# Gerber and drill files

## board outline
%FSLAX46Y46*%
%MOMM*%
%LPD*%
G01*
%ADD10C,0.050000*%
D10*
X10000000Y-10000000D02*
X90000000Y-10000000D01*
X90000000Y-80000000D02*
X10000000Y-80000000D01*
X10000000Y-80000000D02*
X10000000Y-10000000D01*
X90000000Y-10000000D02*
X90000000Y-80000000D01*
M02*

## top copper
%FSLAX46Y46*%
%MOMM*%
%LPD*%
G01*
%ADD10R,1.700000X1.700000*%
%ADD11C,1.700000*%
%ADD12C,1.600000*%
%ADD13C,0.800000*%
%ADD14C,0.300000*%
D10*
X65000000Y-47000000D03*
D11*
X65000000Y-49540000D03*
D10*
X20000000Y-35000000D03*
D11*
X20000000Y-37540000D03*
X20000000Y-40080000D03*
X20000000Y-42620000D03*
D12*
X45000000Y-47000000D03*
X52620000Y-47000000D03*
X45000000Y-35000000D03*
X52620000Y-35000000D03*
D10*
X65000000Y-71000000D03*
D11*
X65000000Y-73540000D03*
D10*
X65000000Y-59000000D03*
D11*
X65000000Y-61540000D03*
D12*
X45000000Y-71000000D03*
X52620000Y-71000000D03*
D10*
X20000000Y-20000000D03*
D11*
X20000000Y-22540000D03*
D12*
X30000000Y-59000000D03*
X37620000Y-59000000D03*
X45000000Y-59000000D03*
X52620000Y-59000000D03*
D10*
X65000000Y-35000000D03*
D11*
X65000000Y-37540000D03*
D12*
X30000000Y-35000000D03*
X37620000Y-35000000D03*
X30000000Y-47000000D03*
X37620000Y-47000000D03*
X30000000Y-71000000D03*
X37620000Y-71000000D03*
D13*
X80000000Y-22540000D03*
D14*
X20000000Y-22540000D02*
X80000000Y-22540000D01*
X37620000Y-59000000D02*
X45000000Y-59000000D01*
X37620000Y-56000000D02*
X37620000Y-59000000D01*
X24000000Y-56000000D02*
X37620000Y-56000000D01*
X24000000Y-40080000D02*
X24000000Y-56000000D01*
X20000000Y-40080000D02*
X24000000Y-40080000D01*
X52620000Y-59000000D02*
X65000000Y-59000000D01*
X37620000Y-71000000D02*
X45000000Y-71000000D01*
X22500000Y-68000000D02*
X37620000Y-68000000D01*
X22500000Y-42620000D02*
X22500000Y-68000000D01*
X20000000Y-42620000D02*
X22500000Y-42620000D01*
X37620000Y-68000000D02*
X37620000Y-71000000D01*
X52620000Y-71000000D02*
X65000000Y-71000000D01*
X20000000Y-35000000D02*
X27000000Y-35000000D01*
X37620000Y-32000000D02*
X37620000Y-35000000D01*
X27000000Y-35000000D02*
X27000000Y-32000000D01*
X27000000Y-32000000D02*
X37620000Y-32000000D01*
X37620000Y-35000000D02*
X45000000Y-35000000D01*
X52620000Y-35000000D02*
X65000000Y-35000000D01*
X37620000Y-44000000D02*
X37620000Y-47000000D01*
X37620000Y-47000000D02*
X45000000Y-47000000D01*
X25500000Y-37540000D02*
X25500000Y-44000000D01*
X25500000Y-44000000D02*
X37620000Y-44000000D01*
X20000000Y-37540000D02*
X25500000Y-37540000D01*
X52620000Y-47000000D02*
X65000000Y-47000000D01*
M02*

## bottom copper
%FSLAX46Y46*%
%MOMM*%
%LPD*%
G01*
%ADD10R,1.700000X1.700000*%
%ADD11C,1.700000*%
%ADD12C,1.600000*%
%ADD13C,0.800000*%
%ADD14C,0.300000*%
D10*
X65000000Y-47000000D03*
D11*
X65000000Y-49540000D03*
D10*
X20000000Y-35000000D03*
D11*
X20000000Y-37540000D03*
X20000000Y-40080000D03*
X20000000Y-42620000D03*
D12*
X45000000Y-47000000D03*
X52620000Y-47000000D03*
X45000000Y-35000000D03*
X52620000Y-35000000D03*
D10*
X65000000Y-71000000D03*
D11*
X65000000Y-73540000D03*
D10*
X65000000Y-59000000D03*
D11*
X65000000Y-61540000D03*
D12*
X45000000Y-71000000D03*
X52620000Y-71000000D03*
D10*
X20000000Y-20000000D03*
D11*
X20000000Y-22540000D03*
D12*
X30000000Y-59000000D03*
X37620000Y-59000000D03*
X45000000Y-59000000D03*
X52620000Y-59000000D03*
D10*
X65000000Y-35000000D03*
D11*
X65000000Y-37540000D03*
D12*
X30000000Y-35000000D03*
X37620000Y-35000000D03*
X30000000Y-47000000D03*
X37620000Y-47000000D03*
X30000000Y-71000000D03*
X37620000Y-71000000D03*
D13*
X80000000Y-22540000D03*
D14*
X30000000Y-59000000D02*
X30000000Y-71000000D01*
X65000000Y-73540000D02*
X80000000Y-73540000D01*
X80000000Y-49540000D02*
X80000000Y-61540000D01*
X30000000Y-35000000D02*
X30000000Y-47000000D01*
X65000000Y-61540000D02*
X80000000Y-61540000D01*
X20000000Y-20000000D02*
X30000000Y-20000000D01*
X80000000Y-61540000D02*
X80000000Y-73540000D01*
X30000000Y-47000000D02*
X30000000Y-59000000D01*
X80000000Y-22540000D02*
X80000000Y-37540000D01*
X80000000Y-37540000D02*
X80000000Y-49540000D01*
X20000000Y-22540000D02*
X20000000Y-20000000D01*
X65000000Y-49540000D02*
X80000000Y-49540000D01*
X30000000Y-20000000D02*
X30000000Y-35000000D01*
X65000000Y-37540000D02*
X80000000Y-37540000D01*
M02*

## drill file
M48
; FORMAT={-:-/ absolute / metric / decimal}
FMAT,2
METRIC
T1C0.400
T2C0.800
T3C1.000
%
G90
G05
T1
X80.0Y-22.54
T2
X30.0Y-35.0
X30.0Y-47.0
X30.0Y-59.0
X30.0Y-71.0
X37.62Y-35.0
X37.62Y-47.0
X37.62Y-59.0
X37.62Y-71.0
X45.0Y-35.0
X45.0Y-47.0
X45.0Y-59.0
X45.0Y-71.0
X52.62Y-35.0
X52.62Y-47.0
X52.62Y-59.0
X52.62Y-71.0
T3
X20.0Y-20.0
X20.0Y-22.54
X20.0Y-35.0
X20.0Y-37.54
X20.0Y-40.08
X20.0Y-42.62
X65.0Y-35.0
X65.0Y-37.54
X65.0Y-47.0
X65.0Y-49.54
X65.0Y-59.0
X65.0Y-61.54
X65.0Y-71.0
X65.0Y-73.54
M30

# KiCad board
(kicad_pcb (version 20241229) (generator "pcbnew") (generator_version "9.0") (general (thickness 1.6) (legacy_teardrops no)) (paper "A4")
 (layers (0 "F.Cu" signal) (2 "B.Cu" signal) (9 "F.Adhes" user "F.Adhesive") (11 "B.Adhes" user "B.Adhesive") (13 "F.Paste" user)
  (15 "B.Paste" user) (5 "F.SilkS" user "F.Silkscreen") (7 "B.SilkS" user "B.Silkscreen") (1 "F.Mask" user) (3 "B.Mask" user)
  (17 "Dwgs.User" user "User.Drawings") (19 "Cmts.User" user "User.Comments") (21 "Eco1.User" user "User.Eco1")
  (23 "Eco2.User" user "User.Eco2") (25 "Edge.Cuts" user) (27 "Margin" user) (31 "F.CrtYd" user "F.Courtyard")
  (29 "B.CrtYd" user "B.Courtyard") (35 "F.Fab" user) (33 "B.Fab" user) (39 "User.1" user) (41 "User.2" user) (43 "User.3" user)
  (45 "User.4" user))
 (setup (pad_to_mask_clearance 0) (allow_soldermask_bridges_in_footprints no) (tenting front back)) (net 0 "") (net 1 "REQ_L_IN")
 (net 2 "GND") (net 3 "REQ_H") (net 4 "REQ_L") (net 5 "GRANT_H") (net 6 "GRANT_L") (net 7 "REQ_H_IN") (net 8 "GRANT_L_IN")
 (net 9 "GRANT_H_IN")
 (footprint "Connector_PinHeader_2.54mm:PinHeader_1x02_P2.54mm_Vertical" (layer "F.Cu") (at 65 47)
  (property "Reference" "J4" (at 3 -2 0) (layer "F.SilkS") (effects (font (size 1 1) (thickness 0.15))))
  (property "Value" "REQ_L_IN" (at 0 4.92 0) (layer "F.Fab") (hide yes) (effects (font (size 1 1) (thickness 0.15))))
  (pad "1" thru_hole rect (at 0 0) (size 1.7 1.7) (drill 1) (layers "*.Cu" "*.Mask") (remove_unused_layers no) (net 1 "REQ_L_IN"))
  (pad "2" thru_hole circle (at 0 2.54) (size 1.7 1.7) (drill 1) (layers "*.Cu" "*.Mask") (remove_unused_layers no) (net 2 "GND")))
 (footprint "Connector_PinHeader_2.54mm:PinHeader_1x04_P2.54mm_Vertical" (layer "F.Cu") (at 20 35)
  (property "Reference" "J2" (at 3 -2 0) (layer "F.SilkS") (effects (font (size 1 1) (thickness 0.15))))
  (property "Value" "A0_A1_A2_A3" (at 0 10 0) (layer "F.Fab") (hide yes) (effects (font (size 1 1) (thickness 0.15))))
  (pad "1" thru_hole rect (at 0 0) (size 1.7 1.7) (drill 1) (layers "*.Cu" "*.Mask") (remove_unused_layers no) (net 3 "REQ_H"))
  (pad "2" thru_hole circle (at 0 2.54) (size 1.7 1.7) (drill 1) (layers "*.Cu" "*.Mask") (remove_unused_layers no) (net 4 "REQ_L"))
  (pad "3" thru_hole circle (at 0 5.08) (size 1.7 1.7) (drill 1) (layers "*.Cu" "*.Mask") (remove_unused_layers no) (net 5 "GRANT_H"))
  (pad "4" thru_hole circle (at 0 7.62) (size 1.7 1.7) (drill 1) (layers "*.Cu" "*.Mask") (remove_unused_layers no) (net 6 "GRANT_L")))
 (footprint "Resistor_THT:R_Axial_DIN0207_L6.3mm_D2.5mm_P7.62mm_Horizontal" (layer "F.Cu") (at 45 47)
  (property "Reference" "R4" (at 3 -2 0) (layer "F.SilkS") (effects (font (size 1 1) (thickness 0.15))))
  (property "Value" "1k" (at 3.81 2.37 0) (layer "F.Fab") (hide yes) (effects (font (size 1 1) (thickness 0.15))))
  (pad "1" thru_hole circle (at 0 0) (size 1.6 1.6) (drill 0.8) (layers "*.Cu" "*.Mask") (remove_unused_layers no) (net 4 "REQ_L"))
  (pad "2" thru_hole circle (at 7.62 0) (size 1.6 1.6) (drill 0.8) (layers "*.Cu" "*.Mask") (remove_unused_layers no) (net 1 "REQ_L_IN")))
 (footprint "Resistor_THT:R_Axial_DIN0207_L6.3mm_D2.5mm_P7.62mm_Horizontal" (layer "F.Cu") (at 45 35)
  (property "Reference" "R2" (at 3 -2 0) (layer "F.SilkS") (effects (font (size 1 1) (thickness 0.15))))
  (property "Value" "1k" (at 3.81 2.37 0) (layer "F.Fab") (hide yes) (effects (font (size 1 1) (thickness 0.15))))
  (pad "1" thru_hole circle (at 0 0) (size 1.6 1.6) (drill 0.8) (layers "*.Cu" "*.Mask") (remove_unused_layers no) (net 3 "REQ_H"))
  (pad "2" thru_hole circle (at 7.62 0) (size 1.6 1.6) (drill 0.8) (layers "*.Cu" "*.Mask") (remove_unused_layers no) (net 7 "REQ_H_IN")))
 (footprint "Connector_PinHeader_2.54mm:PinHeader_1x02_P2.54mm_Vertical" (layer "F.Cu") (at 65 71)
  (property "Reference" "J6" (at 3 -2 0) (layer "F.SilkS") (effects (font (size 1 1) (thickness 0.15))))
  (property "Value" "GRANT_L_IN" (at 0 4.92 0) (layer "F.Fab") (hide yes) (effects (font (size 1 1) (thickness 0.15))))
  (pad "1" thru_hole rect (at 0 0) (size 1.7 1.7) (drill 1) (layers "*.Cu" "*.Mask") (remove_unused_layers no) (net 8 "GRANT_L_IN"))
  (pad "2" thru_hole circle (at 0 2.54) (size 1.7 1.7) (drill 1) (layers "*.Cu" "*.Mask") (remove_unused_layers no) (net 2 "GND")))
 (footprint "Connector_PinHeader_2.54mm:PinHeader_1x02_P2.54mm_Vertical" (layer "F.Cu") (at 65 59)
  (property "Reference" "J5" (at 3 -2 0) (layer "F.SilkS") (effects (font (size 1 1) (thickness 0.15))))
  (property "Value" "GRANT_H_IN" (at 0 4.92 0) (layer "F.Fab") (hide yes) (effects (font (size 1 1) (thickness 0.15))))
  (pad "1" thru_hole rect (at 0 0) (size 1.7 1.7) (drill 1) (layers "*.Cu" "*.Mask") (remove_unused_layers no) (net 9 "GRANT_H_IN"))
  (pad "2" thru_hole circle (at 0 2.54) (size 1.7 1.7) (drill 1) (layers "*.Cu" "*.Mask") (remove_unused_layers no) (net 2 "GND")))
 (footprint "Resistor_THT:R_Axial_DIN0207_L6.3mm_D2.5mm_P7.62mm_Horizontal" (layer "F.Cu") (at 45 71)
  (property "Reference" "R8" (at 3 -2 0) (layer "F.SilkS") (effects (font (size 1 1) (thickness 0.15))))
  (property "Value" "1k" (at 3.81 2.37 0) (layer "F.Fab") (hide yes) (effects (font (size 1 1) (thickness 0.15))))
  (pad "1" thru_hole circle (at 0 0) (size 1.6 1.6) (drill 0.8) (layers "*.Cu" "*.Mask") (remove_unused_layers no) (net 6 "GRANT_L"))
  (pad "2" thru_hole circle (at 7.62 0) (size 1.6 1.6) (drill 0.8) (layers "*.Cu" "*.Mask") (remove_unused_layers no) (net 8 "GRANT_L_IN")))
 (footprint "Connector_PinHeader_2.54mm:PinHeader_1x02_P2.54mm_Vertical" (layer "F.Cu") (at 20 20)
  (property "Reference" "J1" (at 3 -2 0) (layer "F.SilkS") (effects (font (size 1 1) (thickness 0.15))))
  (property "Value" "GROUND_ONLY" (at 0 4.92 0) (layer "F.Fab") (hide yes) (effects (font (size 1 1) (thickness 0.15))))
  (pad "1" thru_hole rect (at 0 0) (size 1.7 1.7) (drill 1) (layers "*.Cu" "*.Mask") (remove_unused_layers no) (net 2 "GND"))
  (pad "2" thru_hole circle (at 0 2.54) (size 1.7 1.7) (drill 1) (layers "*.Cu" "*.Mask") (remove_unused_layers no) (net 2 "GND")))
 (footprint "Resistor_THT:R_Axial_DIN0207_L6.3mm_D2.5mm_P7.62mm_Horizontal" (layer "F.Cu") (at 30 59)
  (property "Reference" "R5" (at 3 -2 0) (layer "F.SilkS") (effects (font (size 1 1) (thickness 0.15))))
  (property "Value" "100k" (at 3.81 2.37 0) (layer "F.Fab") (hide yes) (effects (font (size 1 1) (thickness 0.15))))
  (pad "1" thru_hole circle (at 0 0) (size 1.6 1.6) (drill 0.8) (layers "*.Cu" "*.Mask") (remove_unused_layers no) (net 2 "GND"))
  (pad "2" thru_hole circle (at 7.62 0) (size 1.6 1.6) (drill 0.8) (layers "*.Cu" "*.Mask") (remove_unused_layers no) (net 5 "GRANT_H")))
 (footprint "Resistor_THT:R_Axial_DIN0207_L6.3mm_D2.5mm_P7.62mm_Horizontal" (layer "F.Cu") (at 45 59)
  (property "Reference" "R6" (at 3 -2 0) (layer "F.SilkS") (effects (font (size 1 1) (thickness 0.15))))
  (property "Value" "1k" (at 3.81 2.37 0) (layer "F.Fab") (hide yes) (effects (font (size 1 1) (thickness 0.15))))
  (pad "1" thru_hole circle (at 0 0) (size 1.6 1.6) (drill 0.8) (layers "*.Cu" "*.Mask") (remove_unused_layers no) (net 5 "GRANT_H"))
  (pad "2" thru_hole circle (at 7.62 0) (size 1.6 1.6) (drill 0.8) (layers "*.Cu" "*.Mask") (remove_unused_layers no) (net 9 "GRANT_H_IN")))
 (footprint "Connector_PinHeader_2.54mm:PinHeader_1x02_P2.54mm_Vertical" (layer "F.Cu") (at 65 35)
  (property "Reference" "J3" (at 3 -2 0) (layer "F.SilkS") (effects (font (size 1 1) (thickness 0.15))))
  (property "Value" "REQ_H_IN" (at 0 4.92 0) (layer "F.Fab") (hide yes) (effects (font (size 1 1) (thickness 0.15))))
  (pad "1" thru_hole rect (at 0 0) (size 1.7 1.7) (drill 1) (layers "*.Cu" "*.Mask") (remove_unused_layers no) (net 7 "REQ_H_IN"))
  (pad "2" thru_hole circle (at 0 2.54) (size 1.7 1.7) (drill 1) (layers "*.Cu" "*.Mask") (remove_unused_layers no) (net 2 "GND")))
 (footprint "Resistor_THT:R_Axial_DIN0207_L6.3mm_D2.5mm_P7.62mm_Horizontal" (layer "F.Cu") (at 30 35)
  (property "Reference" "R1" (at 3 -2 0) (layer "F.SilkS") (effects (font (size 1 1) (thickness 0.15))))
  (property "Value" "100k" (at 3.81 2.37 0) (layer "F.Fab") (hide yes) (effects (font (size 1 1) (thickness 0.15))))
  (pad "1" thru_hole circle (at 0 0) (size 1.6 1.6) (drill 0.8) (layers "*.Cu" "*.Mask") (remove_unused_layers no) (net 2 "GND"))
  (pad "2" thru_hole circle (at 7.62 0) (size 1.6 1.6) (drill 0.8) (layers "*.Cu" "*.Mask") (remove_unused_layers no) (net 3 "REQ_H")))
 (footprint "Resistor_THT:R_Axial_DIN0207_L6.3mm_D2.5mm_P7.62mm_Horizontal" (layer "F.Cu") (at 30 47)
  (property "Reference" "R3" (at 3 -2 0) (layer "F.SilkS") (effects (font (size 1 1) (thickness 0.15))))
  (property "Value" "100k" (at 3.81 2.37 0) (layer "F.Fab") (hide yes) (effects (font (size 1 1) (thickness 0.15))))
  (pad "1" thru_hole circle (at 0 0) (size 1.6 1.6) (drill 0.8) (layers "*.Cu" "*.Mask") (remove_unused_layers no) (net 2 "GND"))
  (pad "2" thru_hole circle (at 7.62 0) (size 1.6 1.6) (drill 0.8) (layers "*.Cu" "*.Mask") (remove_unused_layers no) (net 4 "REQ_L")))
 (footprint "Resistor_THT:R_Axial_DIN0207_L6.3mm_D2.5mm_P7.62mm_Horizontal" (layer "F.Cu") (at 30 71)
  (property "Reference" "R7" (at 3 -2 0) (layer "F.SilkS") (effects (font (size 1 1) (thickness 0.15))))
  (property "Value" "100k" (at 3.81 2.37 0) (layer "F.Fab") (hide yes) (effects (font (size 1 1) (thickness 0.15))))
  (pad "1" thru_hole circle (at 0 0) (size 1.6 1.6) (drill 0.8) (layers "*.Cu" "*.Mask") (remove_unused_layers no) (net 2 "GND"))
  (pad "2" thru_hole circle (at 7.62 0) (size 1.6 1.6) (drill 0.8) (layers "*.Cu" "*.Mask") (remove_unused_layers no) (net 6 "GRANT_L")))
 (gr_line (start 10 10) (end 90 10) (stroke (width 0.05) (type default)) (layer "Edge.Cuts"))
 (gr_line (start 90 80) (end 10 80) (stroke (width 0.05) (type default)) (layer "Edge.Cuts"))
 (gr_line (start 10 80) (end 10 10) (stroke (width 0.05) (type default)) (layer "Edge.Cuts"))
 (gr_line (start 90 10) (end 90 80) (stroke (width 0.05) (type default)) (layer "Edge.Cuts"))
 (segment (start 20 22.54) (end 80 22.54) (width 0.3) (layer "F.Cu") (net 2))
 (via (at 80 22.54) (size 0.8) (drill 0.4) (layers "F.Cu" "B.Cu") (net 2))
 (segment (start 30 59) (end 30 71) (width 0.3) (layer "B.Cu") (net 2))
 (segment (start 65 73.54) (end 80 73.54) (width 0.3) (layer "B.Cu") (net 2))
 (segment (start 80 49.54) (end 80 61.54) (width 0.3) (layer "B.Cu") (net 2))
 (segment (start 30 35) (end 30 47) (width 0.3) (layer "B.Cu") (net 2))
 (segment (start 65 61.54) (end 80 61.54) (width 0.3) (layer "B.Cu") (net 2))
 (segment (start 20 20) (end 30 20) (width 0.3) (layer "B.Cu") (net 2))
 (segment (start 80 61.54) (end 80 73.54) (width 0.3) (layer "B.Cu") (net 2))
 (segment (start 30 47) (end 30 59) (width 0.3) (layer "B.Cu") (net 2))
 (segment (start 80 22.54) (end 80 37.54) (width 0.3) (layer "B.Cu") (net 2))
 (segment (start 80 37.54) (end 80 49.54) (width 0.3) (layer "B.Cu") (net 2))
 (segment (start 20 22.54) (end 20 20) (width 0.3) (layer "B.Cu") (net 2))
 (segment (start 65 49.54) (end 80 49.54) (width 0.3) (layer "B.Cu") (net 2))
 (segment (start 30 20) (end 30 35) (width 0.3) (layer "B.Cu") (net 2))
 (segment (start 65 37.54) (end 80 37.54) (width 0.3) (layer "B.Cu") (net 2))
 (segment (start 37.62 59) (end 45 59) (width 0.3) (layer "F.Cu") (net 5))
 (segment (start 37.62 56) (end 37.62 59) (width 0.3) (layer "F.Cu") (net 5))
 (segment (start 24 56) (end 37.62 56) (width 0.3) (layer "F.Cu") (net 5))
 (segment (start 24 40.08) (end 24 56) (width 0.3) (layer "F.Cu") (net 5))
 (segment (start 20 40.08) (end 24 40.08) (width 0.3) (layer "F.Cu") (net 5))
 (segment (start 52.62 59) (end 65 59) (width 0.3) (layer "F.Cu") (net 9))
 (segment (start 37.62 71) (end 45 71) (width 0.3) (layer "F.Cu") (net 6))
 (segment (start 22.5 68) (end 37.62 68) (width 0.3) (layer "F.Cu") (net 6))
 (segment (start 22.5 42.62) (end 22.5 68) (width 0.3) (layer "F.Cu") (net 6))
 (segment (start 20 42.62) (end 22.5 42.62) (width 0.3) (layer "F.Cu") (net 6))
 (segment (start 37.62 68) (end 37.62 71) (width 0.3) (layer "F.Cu") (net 6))
 (segment (start 52.62 71) (end 65 71) (width 0.3) (layer "F.Cu") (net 8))
 (segment (start 20 35) (end 27 35) (width 0.3) (layer "F.Cu") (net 3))
 (segment (start 37.62 32) (end 37.62 35) (width 0.3) (layer "F.Cu") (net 3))
 (segment (start 27 35) (end 27 32) (width 0.3) (layer "F.Cu") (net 3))
 (segment (start 27 32) (end 37.62 32) (width 0.3) (layer "F.Cu") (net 3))
 (segment (start 37.62 35) (end 45 35) (width 0.3) (layer "F.Cu") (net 3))
 (segment (start 52.62 35) (end 65 35) (width 0.3) (layer "F.Cu") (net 7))
 (segment (start 37.62 44) (end 37.62 47) (width 0.3) (layer "F.Cu") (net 4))
 (segment (start 37.62 47) (end 45 47) (width 0.3) (layer "F.Cu") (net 4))
 (segment (start 25.5 37.54) (end 25.5 44) (width 0.3) (layer "F.Cu") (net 4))
 (segment (start 25.5 44) (end 37.62 44) (width 0.3) (layer "F.Cu") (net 4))
 (segment (start 20 37.54) (end 25.5 37.54) (width 0.3) (layer "F.Cu") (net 4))
 (segment (start 52.62 47) (end 65 47) (width 0.3) (layer "F.Cu") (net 1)))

